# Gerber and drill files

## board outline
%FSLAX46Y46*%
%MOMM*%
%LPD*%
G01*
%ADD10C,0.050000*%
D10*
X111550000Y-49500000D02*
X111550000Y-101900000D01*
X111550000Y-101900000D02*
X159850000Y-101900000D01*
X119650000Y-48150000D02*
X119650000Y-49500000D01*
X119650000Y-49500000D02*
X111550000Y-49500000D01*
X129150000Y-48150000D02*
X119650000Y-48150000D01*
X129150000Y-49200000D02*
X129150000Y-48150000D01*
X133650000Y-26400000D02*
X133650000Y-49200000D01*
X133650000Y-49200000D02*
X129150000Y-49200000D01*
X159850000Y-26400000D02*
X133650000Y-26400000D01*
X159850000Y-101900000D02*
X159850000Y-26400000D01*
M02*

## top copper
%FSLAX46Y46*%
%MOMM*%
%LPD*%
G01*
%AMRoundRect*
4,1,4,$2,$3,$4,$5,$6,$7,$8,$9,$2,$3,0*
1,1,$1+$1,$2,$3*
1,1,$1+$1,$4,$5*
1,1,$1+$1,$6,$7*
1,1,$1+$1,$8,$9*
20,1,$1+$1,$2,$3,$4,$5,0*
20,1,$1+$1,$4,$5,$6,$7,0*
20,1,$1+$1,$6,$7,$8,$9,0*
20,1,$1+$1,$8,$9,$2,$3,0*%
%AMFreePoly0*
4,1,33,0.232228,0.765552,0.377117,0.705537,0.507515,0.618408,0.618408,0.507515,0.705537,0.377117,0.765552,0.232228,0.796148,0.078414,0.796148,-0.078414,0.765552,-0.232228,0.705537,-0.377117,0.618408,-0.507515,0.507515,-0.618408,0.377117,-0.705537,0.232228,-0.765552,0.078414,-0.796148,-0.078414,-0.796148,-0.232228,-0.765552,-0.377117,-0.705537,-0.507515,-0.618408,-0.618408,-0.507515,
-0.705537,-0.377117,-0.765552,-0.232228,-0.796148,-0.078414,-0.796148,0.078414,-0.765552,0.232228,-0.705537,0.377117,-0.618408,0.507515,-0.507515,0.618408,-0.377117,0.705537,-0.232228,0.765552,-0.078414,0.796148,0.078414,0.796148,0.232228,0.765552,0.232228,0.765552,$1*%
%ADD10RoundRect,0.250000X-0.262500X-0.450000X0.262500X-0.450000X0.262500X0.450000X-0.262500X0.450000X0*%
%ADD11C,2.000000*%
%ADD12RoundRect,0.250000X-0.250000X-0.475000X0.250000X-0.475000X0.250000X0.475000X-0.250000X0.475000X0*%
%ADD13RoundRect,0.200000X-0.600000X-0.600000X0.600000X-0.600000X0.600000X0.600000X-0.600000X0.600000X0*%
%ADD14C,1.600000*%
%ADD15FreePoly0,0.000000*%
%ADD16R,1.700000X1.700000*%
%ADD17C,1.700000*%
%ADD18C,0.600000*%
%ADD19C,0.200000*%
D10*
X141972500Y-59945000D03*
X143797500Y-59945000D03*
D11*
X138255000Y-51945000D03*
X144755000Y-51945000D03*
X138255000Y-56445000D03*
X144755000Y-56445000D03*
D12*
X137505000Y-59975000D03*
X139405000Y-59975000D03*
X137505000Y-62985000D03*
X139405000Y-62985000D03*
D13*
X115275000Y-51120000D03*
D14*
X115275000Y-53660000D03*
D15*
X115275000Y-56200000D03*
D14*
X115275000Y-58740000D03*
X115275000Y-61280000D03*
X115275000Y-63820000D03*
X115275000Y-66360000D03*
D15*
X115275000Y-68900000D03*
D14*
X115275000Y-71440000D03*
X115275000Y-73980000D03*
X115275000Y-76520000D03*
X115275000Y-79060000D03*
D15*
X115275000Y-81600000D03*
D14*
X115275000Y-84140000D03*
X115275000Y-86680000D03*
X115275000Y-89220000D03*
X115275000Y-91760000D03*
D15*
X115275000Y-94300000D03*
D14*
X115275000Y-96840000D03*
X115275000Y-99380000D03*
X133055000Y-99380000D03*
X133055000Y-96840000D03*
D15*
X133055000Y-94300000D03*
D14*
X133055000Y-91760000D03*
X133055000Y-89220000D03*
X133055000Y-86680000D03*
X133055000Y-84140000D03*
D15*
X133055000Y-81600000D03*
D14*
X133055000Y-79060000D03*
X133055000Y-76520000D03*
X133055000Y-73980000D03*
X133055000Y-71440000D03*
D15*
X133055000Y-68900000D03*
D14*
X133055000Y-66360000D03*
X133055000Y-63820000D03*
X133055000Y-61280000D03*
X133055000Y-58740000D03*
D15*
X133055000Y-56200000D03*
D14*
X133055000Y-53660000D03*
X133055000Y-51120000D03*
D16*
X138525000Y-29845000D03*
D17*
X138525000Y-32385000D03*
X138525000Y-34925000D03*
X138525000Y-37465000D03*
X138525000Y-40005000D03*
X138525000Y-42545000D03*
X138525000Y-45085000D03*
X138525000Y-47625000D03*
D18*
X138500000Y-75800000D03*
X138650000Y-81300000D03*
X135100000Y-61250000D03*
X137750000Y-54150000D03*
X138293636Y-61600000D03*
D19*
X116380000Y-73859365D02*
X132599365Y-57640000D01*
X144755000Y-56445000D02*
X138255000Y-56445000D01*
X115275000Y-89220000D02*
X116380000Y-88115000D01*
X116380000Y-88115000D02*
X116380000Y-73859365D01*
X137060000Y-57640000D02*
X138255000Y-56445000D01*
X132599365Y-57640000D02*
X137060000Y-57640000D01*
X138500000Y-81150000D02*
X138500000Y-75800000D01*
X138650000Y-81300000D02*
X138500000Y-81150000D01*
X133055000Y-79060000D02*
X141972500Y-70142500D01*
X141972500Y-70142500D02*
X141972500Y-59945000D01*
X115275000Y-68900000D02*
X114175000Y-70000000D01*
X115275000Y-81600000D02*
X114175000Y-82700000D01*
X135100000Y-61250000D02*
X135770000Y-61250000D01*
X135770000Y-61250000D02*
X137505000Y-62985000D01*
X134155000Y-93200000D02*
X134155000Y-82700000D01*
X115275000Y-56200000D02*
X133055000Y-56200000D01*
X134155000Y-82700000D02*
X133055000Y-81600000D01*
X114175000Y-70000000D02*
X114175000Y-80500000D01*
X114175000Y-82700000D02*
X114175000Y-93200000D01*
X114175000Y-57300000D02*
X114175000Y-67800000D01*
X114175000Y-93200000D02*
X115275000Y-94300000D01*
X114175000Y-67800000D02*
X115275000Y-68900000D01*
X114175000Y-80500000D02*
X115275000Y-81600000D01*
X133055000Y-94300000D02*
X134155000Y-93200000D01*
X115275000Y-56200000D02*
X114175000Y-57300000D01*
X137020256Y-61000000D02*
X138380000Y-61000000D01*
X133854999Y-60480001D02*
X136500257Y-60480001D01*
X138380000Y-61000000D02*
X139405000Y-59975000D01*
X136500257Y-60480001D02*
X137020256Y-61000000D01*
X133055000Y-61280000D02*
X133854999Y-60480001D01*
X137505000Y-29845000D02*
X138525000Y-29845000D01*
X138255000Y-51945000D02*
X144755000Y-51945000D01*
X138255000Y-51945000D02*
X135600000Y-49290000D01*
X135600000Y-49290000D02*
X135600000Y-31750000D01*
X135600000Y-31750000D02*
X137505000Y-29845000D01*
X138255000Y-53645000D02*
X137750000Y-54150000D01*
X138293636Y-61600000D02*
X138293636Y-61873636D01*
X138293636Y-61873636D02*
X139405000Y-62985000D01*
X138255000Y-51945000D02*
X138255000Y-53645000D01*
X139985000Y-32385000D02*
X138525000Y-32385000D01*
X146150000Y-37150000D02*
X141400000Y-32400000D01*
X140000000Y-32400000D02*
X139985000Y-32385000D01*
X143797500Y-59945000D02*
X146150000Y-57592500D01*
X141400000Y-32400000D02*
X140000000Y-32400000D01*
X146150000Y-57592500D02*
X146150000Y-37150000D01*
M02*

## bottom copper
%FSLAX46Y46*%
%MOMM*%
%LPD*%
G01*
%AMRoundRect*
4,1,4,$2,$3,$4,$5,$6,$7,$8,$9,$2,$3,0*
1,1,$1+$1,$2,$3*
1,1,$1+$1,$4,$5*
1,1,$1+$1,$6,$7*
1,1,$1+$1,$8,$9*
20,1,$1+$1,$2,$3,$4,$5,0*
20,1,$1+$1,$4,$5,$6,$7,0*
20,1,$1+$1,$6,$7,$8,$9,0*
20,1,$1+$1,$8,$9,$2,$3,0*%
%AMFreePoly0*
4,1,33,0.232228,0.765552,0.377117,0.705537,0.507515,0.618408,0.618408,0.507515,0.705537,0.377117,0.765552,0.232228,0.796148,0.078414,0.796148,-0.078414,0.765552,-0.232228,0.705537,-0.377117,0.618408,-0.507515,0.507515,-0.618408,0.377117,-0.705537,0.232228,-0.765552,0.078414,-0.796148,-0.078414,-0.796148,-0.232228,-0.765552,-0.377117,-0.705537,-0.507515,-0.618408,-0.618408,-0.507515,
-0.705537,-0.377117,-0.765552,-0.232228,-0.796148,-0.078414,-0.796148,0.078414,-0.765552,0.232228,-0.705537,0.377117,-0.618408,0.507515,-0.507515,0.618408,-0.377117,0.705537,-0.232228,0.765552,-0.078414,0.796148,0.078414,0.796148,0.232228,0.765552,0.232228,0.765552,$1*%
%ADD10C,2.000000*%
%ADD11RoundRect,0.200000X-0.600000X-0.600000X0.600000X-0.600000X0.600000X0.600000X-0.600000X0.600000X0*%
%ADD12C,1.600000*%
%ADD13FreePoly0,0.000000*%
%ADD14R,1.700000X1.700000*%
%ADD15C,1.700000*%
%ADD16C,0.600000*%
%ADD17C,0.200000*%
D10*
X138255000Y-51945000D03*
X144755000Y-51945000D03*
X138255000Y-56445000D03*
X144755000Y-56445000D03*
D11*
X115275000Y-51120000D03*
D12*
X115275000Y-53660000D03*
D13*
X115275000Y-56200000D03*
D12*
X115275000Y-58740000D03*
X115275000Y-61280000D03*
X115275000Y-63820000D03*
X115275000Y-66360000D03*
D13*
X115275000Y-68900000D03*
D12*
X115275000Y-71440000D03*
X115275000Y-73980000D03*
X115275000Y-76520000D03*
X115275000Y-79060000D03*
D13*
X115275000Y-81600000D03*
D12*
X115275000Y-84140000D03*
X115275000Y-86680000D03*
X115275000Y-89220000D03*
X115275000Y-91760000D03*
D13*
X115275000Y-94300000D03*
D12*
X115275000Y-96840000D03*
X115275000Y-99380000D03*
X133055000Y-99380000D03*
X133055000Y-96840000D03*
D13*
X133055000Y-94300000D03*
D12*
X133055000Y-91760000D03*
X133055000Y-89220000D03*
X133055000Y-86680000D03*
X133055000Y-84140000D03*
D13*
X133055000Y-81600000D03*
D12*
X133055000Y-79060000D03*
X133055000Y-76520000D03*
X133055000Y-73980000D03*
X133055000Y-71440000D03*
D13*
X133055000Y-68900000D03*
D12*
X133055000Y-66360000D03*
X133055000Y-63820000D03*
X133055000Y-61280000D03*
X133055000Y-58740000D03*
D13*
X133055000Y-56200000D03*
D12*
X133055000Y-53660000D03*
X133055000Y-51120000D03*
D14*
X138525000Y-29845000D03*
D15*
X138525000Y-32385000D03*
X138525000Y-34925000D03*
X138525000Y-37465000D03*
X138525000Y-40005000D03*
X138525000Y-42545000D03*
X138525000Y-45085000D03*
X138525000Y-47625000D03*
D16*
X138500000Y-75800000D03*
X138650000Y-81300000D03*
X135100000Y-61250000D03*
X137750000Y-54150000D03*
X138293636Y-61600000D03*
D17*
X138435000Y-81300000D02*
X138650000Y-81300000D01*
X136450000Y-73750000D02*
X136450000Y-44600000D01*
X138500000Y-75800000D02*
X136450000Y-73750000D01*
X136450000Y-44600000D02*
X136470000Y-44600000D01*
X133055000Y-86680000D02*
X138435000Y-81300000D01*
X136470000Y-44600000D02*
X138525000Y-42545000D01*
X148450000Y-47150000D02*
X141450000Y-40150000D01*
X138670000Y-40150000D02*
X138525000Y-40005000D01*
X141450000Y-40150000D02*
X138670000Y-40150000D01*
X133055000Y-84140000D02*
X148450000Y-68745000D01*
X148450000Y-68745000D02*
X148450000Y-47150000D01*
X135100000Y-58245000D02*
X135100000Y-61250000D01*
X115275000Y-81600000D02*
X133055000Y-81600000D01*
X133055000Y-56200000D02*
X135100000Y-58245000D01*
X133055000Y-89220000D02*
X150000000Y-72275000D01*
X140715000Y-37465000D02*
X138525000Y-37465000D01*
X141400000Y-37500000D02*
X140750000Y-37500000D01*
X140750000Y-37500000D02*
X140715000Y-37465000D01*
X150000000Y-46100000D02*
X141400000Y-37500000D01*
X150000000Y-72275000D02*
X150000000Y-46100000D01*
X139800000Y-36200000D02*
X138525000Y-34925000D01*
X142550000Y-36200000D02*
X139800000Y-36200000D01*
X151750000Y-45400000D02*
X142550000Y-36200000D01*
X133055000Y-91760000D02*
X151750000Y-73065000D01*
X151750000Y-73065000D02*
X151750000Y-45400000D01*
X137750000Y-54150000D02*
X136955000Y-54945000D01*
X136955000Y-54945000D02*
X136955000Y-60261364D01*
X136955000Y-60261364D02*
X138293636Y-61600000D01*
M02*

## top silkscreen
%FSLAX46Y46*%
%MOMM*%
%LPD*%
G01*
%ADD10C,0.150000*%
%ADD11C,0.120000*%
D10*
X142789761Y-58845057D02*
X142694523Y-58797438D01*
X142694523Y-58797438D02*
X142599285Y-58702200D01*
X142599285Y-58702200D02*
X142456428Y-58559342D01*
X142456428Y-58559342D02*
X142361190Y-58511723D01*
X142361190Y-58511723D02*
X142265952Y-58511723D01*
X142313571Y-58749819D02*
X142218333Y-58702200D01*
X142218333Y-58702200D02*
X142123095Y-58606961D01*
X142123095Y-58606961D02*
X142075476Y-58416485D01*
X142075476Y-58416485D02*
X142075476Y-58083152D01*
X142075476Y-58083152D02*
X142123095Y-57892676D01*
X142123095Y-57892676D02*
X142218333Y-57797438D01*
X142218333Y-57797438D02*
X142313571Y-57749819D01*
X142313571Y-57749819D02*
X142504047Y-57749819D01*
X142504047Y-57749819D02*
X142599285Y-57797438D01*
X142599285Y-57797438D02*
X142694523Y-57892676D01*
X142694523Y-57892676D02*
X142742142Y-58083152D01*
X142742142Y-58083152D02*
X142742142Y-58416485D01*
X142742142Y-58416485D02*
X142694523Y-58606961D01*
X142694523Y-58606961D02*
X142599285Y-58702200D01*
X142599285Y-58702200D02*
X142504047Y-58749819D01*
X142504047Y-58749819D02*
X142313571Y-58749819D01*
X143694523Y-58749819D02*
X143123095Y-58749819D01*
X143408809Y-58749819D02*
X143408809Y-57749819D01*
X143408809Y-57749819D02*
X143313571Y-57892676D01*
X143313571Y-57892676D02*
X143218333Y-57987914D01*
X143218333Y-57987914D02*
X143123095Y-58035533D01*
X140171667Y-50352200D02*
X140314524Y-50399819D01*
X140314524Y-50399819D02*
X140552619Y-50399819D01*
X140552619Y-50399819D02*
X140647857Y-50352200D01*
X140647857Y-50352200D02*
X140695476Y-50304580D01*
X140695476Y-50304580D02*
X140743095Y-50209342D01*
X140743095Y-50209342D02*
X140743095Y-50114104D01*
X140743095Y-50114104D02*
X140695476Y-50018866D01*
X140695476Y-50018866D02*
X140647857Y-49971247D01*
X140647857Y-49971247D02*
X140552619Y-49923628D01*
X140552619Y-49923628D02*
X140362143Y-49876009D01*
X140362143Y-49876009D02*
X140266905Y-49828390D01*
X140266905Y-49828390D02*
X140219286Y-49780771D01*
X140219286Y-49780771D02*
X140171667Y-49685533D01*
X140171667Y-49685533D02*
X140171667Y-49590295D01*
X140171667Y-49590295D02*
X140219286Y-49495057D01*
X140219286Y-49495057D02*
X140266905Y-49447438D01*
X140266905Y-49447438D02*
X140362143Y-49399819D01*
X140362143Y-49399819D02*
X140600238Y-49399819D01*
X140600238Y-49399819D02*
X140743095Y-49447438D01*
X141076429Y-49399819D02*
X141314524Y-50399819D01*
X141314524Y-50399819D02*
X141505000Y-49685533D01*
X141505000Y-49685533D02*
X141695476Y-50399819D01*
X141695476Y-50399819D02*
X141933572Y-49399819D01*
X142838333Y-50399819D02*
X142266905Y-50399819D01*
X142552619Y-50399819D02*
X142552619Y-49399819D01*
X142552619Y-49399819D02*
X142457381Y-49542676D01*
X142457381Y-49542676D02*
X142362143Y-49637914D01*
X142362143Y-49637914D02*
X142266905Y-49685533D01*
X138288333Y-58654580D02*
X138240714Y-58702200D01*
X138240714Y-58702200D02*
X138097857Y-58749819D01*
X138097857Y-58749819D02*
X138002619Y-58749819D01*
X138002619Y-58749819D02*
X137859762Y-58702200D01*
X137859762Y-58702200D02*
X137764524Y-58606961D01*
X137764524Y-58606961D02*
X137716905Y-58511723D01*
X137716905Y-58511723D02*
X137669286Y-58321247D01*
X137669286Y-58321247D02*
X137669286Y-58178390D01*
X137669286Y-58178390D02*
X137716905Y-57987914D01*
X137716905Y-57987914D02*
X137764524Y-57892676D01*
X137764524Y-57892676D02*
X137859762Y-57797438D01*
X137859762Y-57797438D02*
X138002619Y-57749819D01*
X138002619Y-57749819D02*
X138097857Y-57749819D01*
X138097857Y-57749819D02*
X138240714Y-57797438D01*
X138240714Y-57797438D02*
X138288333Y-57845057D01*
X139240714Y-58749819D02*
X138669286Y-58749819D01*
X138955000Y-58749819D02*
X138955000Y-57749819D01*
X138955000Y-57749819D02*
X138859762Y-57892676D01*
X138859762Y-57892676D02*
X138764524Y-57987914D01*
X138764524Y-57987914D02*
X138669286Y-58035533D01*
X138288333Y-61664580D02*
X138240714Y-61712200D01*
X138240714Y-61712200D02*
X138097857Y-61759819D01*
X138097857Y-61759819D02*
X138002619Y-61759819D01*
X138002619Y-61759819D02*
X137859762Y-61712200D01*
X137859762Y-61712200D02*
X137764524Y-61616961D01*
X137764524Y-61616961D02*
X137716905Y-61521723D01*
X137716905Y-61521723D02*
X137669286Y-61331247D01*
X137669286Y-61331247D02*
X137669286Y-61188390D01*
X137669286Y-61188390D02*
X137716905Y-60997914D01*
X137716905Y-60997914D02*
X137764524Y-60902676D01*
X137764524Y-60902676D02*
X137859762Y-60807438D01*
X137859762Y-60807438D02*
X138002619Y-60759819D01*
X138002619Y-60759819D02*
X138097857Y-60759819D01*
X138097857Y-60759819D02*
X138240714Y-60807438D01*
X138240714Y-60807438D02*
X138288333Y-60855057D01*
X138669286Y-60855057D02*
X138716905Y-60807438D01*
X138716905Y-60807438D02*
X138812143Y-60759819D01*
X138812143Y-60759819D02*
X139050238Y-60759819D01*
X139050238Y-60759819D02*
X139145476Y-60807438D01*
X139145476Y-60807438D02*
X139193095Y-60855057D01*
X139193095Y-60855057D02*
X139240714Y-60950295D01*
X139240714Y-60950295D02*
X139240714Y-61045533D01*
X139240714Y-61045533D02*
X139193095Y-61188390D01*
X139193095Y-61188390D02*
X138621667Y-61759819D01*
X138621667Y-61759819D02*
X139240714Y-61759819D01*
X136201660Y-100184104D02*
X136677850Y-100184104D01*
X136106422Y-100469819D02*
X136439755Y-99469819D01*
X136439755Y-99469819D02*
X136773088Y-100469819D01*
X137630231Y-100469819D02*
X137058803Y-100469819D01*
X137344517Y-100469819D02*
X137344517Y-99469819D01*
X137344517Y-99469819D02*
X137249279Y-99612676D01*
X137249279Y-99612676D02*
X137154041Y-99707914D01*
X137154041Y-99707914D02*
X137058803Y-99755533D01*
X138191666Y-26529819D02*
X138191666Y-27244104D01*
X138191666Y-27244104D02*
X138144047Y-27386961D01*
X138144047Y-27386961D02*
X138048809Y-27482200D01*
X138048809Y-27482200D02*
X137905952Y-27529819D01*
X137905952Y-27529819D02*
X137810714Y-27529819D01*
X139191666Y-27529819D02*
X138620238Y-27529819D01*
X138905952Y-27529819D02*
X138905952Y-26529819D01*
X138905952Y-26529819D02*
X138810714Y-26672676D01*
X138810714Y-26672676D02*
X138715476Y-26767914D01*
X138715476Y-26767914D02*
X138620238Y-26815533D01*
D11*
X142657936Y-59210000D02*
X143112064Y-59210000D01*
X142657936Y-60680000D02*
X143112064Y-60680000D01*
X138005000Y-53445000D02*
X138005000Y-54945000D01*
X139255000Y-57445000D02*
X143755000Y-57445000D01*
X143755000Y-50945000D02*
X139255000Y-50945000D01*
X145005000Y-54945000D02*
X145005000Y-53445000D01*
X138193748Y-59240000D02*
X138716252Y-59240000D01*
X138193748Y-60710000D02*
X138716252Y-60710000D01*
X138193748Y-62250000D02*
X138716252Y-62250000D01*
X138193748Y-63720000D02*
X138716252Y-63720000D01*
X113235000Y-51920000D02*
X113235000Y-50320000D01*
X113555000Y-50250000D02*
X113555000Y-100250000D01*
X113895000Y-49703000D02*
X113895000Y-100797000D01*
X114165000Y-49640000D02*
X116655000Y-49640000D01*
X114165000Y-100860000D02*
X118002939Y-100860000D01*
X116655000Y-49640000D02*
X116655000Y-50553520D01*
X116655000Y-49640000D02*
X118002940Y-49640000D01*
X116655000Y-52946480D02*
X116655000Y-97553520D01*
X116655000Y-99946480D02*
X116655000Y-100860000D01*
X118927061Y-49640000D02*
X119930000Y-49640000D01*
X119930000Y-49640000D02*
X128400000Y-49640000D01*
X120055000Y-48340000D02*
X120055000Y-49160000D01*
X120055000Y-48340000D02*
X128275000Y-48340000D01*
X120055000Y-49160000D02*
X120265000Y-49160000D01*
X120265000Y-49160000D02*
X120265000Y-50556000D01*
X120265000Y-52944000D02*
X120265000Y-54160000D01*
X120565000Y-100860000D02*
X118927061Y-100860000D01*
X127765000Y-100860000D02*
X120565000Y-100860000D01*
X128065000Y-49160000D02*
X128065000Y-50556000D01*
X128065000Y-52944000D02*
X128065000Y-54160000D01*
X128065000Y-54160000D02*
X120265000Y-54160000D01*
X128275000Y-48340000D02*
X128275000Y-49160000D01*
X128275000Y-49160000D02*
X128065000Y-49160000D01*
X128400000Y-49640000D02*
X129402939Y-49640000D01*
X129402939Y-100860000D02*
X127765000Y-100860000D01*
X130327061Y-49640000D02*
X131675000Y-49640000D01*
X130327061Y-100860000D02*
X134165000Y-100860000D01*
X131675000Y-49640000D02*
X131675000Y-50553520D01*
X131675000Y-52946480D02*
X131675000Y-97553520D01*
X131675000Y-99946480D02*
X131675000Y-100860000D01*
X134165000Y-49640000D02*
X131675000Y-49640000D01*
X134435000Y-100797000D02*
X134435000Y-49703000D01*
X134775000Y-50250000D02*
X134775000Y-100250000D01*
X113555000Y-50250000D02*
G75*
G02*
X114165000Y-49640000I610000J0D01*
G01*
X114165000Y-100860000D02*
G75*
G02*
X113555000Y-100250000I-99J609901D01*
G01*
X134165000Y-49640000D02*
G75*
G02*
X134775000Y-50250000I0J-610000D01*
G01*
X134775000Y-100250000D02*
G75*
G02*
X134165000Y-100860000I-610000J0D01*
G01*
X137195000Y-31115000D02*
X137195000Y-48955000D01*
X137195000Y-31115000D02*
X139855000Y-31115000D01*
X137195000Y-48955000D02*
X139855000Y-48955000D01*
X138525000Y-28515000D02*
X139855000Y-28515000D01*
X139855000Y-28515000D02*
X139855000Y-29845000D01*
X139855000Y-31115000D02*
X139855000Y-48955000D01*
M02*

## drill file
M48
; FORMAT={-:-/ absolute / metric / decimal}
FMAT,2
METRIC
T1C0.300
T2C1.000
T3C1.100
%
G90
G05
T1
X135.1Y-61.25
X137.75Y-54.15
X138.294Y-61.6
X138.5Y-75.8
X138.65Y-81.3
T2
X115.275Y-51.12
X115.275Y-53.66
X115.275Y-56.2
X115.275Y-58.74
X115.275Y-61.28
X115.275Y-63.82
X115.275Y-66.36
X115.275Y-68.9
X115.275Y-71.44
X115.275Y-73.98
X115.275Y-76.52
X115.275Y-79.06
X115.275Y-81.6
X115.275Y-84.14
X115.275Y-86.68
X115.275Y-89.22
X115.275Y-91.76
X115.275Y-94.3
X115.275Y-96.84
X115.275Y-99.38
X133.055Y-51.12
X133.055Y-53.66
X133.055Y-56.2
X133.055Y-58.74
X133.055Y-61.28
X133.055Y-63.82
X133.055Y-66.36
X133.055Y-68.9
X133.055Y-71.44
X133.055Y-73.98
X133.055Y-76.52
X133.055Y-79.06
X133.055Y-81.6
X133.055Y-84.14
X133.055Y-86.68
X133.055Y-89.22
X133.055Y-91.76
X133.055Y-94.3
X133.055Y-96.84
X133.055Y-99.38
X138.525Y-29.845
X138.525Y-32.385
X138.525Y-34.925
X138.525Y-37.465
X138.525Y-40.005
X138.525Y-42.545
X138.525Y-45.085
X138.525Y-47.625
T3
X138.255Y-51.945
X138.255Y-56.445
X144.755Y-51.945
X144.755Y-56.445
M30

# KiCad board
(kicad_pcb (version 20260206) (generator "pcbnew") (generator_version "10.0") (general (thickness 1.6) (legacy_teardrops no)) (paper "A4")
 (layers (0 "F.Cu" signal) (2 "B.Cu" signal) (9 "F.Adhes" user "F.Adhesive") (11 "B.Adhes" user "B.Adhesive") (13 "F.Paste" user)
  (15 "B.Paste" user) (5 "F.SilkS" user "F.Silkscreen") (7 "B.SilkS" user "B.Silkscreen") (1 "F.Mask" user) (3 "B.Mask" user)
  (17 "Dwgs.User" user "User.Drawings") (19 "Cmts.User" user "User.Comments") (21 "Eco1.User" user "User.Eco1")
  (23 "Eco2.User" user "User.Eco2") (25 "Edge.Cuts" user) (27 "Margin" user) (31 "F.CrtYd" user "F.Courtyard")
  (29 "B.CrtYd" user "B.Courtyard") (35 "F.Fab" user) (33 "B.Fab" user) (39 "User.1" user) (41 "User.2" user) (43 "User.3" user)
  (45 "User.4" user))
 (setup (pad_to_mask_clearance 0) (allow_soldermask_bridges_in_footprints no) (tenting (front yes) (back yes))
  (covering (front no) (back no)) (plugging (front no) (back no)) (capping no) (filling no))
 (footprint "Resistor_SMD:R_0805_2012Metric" (layer "F.Cu") (at 142.885 59.945)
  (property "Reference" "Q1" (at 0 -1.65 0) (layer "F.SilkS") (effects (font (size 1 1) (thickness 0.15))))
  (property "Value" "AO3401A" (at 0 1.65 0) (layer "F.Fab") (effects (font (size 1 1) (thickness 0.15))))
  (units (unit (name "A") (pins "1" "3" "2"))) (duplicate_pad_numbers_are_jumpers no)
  (fp_line (start -0.227064 -0.735) (end 0.227064 -0.735) (stroke (width 0.12) (type solid)) (layer "F.SilkS"))
  (fp_line (start -0.227064 0.735) (end 0.227064 0.735) (stroke (width 0.12) (type solid)) (layer "F.SilkS"))
  (pad "1" smd roundrect (at -0.9125 0) (size 1.025 1.4) (layers "F.Cu" "F.Mask" "F.Paste") (roundrect_rratio 0.243902) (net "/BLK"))
  (pad "2" smd roundrect (at 0.9125 0) (size 1.025 1.4) (layers "F.Cu" "F.Mask" "F.Paste") (roundrect_rratio 0.243902) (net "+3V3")))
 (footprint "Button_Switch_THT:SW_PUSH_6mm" (layer "F.Cu") (at 138.255 51.945)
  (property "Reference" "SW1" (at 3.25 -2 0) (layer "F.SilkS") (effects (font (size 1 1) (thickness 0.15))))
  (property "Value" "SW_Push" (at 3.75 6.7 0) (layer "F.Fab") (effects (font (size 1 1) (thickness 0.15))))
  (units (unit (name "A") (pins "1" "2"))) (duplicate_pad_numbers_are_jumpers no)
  (fp_line (start -0.25 1.5) (end -0.25 3) (stroke (width 0.12) (type solid)) (layer "F.SilkS"))
  (fp_line (start 1 5.5) (end 5.5 5.5) (stroke (width 0.12) (type solid)) (layer "F.SilkS"))
  (fp_line (start 5.5 -1) (end 1 -1) (stroke (width 0.12) (type solid)) (layer "F.SilkS"))
  (fp_line (start 6.75 3) (end 6.75 1.5) (stroke (width 0.12) (type solid)) (layer "F.SilkS"))
  (pad "1" thru_hole circle (at 0 0 90) (size 2 2) (drill 1.1) (layers "*.Cu" "*.Mask") (remove_unused_layers no) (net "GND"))
  (pad "1" thru_hole circle (at 6.5 0 90) (size 2 2) (drill 1.1) (layers "*.Cu" "*.Mask") (remove_unused_layers no) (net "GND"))
  (pad "2" thru_hole circle (at 0 4.5 90) (size 2 2) (drill 1.1) (layers "*.Cu" "*.Mask") (remove_unused_layers no) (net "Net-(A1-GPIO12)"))
  (pad "2" thru_hole circle (at 6.5 4.5 90) (size 2 2) (drill 1.1) (layers "*.Cu" "*.Mask") (remove_unused_layers no)
   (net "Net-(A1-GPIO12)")))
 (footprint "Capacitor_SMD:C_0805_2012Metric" (layer "F.Cu") (at 138.455 59.975)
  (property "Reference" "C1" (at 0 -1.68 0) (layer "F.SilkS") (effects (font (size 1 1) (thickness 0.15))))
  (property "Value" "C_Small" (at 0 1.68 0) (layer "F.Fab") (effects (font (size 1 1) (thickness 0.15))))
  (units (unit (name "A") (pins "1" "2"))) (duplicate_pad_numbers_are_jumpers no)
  (fp_line (start -0.261252 -0.735) (end 0.261252 -0.735) (stroke (width 0.12) (type solid)) (layer "F.SilkS"))
  (fp_line (start -0.261252 0.735) (end 0.261252 0.735) (stroke (width 0.12) (type solid)) (layer "F.SilkS"))
  (pad "1" smd roundrect (at -0.95 0) (size 1 1.45) (layers "F.Cu" "F.Mask" "F.Paste") (roundrect_rratio 0.25) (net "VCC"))
  (pad "2" smd roundrect (at 0.95 0) (size 1 1.45) (layers "F.Cu" "F.Mask" "F.Paste") (roundrect_rratio 0.25) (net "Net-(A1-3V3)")))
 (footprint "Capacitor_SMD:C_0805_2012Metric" (layer "F.Cu") (at 138.455 62.985)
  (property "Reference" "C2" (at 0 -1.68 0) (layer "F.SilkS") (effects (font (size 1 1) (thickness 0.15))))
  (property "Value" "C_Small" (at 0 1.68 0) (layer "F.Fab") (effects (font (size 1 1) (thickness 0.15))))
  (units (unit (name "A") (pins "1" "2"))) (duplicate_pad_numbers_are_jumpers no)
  (fp_line (start -0.261252 -0.735) (end 0.261252 -0.735) (stroke (width 0.12) (type solid)) (layer "F.SilkS"))
  (fp_line (start -0.261252 0.735) (end 0.261252 0.735) (stroke (width 0.12) (type solid)) (layer "F.SilkS"))
  (pad "1" smd roundrect (at -0.95 0) (size 1 1.45) (layers "F.Cu" "F.Mask" "F.Paste") (roundrect_rratio 0.25) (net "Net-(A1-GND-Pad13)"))
  (pad "2" smd roundrect (at 0.95 0) (size 1 1.45) (layers "F.Cu" "F.Mask" "F.Paste") (roundrect_rratio 0.25) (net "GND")))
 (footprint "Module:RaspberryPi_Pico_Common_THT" (layer "F.Cu") (at 115.275 51.12)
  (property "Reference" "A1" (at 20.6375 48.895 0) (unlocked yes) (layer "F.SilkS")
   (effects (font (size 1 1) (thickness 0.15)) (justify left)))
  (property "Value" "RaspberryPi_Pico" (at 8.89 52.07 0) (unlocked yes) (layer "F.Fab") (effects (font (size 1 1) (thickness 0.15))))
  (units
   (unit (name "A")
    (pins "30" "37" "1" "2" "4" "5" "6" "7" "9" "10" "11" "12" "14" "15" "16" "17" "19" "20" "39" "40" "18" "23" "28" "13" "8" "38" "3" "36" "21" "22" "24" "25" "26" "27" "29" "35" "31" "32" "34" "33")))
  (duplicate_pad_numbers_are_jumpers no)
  (fp_line (start -2.04 0.8) (end -2.04 -0.8) (stroke (width 0.12) (type solid)) (layer "F.SilkS"))
  (fp_line (start -1.72 -0.87) (end -1.72 49.13) (stroke (width 0.12) (type solid)) (layer "F.SilkS"))
  (fp_line (start -1.38 -1.417) (end -1.38 49.677) (stroke (width 0.12) (type solid)) (layer "F.SilkS"))
  (fp_line (start -1.11 -1.48) (end 1.38 -1.48) (stroke (width 0.12) (type solid)) (layer "F.SilkS"))
  (fp_line (start -1.11 49.74) (end 2.727939 49.74) (stroke (width 0.12) (type solid)) (layer "F.SilkS"))
  (fp_line (start 1.38 -1.48) (end 1.38 -0.56648) (stroke (width 0.12) (type solid)) (layer "F.SilkS"))
  (fp_line (start 1.38 -1.48) (end 2.72794 -1.48) (stroke (width 0.12) (type solid)) (layer "F.SilkS"))
  (fp_line (start 1.38 1.82648) (end 1.38 46.43352) (stroke (width 0.12) (type solid)) (layer "F.SilkS"))
  (fp_line (start 1.38 48.82648) (end 1.38 49.74) (stroke (width 0.12) (type solid)) (layer "F.SilkS"))
  (fp_line (start 3.652061 -1.48) (end 4.655 -1.48) (stroke (width 0.12) (type solid)) (layer "F.SilkS"))
  (fp_line (start 4.655 -1.48) (end 13.125 -1.48) (stroke (width 0.12) (type solid)) (layer "F.SilkS"))
  (fp_line (start 4.78 -2.78) (end 4.78 -1.96) (stroke (width 0.12) (type solid)) (layer "F.SilkS"))
  (fp_line (start 4.78 -2.78) (end 13 -2.78) (stroke (width 0.12) (type solid)) (layer "F.SilkS"))
  (fp_line (start 4.78 -1.96) (end 4.99 -1.96) (stroke (width 0.12) (type solid)) (layer "F.SilkS"))
  (fp_line (start 4.99 -1.96) (end 4.99 -0.564) (stroke (width 0.12) (type solid)) (layer "F.SilkS"))
  (fp_line (start 4.99 1.824) (end 4.99 3.04) (stroke (width 0.12) (type solid)) (layer "F.SilkS"))
  (fp_line (start 5.29 49.74) (end 3.652061 49.74) (stroke (width 0.12) (type solid)) (layer "F.SilkS"))
  (fp_line (start 12.49 49.74) (end 5.29 49.74) (stroke (width 0.12) (type solid)) (layer "F.SilkS"))
  (fp_line (start 12.79 -1.96) (end 12.79 -0.564) (stroke (width 0.12) (type solid)) (layer "F.SilkS"))
  (fp_line (start 12.79 1.824) (end 12.79 3.04) (stroke (width 0.12) (type solid)) (layer "F.SilkS"))
  (fp_line (start 12.79 3.04) (end 4.99 3.04) (stroke (width 0.12) (type solid)) (layer "F.SilkS"))
  (fp_line (start 13 -2.78) (end 13 -1.96) (stroke (width 0.12) (type solid)) (layer "F.SilkS"))
  (fp_line (start 13 -1.96) (end 12.79 -1.96) (stroke (width 0.12) (type solid)) (layer "F.SilkS"))
  (fp_line (start 13.125 -1.48) (end 14.127939 -1.48) (stroke (width 0.12) (type solid)) (layer "F.SilkS"))
  (fp_line (start 14.127939 49.74) (end 12.49 49.74) (stroke (width 0.12) (type solid)) (layer "F.SilkS"))
  (fp_line (start 15.052061 -1.48) (end 16.4 -1.48) (stroke (width 0.12) (type solid)) (layer "F.SilkS"))
  (fp_line (start 15.052061 49.74) (end 18.89 49.74) (stroke (width 0.12) (type solid)) (layer "F.SilkS"))
  (fp_line (start 16.4 -1.48) (end 16.4 -0.56648) (stroke (width 0.12) (type solid)) (layer "F.SilkS"))
  (fp_line (start 16.4 1.82648) (end 16.4 46.43352) (stroke (width 0.12) (type solid)) (layer "F.SilkS"))
  (fp_line (start 16.4 48.82648) (end 16.4 49.74) (stroke (width 0.12) (type solid)) (layer "F.SilkS"))
  (fp_line (start 18.89 -1.48) (end 16.4 -1.48) (stroke (width 0.12) (type solid)) (layer "F.SilkS"))
  (fp_line (start 19.16 49.677) (end 19.16 -1.417) (stroke (width 0.12) (type solid)) (layer "F.SilkS"))
  (fp_line (start 19.5 -0.87) (end 19.5 49.13) (stroke (width 0.12) (type solid)) (layer "F.SilkS"))
  (fp_arc (start -1.72 -0.87) (mid -1.541335 -1.301335) (end -1.11 -1.48) (stroke (width 0.12) (type solid)) (layer "F.SilkS"))
  (fp_arc (start -1.11 49.74) (mid -1.541364 49.561364) (end -1.72 49.13) (stroke (width 0.12) (type solid)) (layer "F.SilkS"))
  (fp_arc (start 18.89 -1.48) (mid 19.321335 -1.301335) (end 19.5 -0.87) (stroke (width 0.12) (type solid)) (layer "F.SilkS"))
  (fp_arc (start 19.5 49.13) (mid 19.321335 49.561335) (end 18.89 49.74) (stroke (width 0.12) (type solid)) (layer "F.SilkS"))
  (pad "1" thru_hole roundrect (at 0 0) (size 1.6 1.6) (drill 1) (layers "*.Cu" "*.Mask") (remove_unused_layers no) (roundrect_rratio 0.125)
   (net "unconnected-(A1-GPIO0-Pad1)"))
  (pad "2" thru_hole circle (at 0 2.54) (size 1.6 1.6) (drill 1) (layers "*.Cu" "*.Mask") (remove_unused_layers no)
   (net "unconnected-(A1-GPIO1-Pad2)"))
  (pad "3" thru_hole custom (at 0 5.08) (size 1.6 1.6) (drill 1) (layers "*.Cu" "*.Mask") (remove_unused_layers no)
   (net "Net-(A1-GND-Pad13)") (options (clearance outline) (anchor circle)) (primitives))
  (pad "4" thru_hole circle (at 0 7.62) (size 1.6 1.6) (drill 1) (layers "*.Cu" "*.Mask") (remove_unused_layers no)
   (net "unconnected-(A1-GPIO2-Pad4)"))
  (pad "5" thru_hole circle (at 0 10.16) (size 1.6 1.6) (drill 1) (layers "*.Cu" "*.Mask") (remove_unused_layers no)
   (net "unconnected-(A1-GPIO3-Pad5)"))
  (pad "6" thru_hole circle (at 0 12.7) (size 1.6 1.6) (drill 1) (layers "*.Cu" "*.Mask") (remove_unused_layers no)
   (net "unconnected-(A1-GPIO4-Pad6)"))
  (pad "7" thru_hole circle (at 0 15.24) (size 1.6 1.6) (drill 1) (layers "*.Cu" "*.Mask") (remove_unused_layers no)
   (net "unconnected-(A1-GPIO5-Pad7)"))
  (pad "8" thru_hole custom (at 0 17.78) (size 1.6 1.6) (drill 1) (layers "*.Cu" "*.Mask") (remove_unused_layers no)
   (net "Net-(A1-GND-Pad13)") (options (clearance outline) (anchor circle)) (primitives))
  (pad "9" thru_hole circle (at 0 20.32) (size 1.6 1.6) (drill 1) (layers "*.Cu" "*.Mask") (remove_unused_layers no)
   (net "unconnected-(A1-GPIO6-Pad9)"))
  (pad "10" thru_hole circle (at 0 22.86) (size 1.6 1.6) (drill 1) (layers "*.Cu" "*.Mask") (remove_unused_layers no)
   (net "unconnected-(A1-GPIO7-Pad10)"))
  (pad "11" thru_hole circle (at 0 25.4) (size 1.6 1.6) (drill 1) (layers "*.Cu" "*.Mask") (remove_unused_layers no)
   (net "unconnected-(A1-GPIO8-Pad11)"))
  (pad "12" thru_hole circle (at 0 27.94) (size 1.6 1.6) (drill 1) (layers "*.Cu" "*.Mask") (remove_unused_layers no)
   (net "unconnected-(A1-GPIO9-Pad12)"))
  (pad "13" thru_hole custom (at 0 30.48) (size 1.6 1.6) (drill 1) (layers "*.Cu" "*.Mask") (remove_unused_layers no)
   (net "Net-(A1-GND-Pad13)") (options (clearance outline) (anchor circle)) (primitives))
  (pad "14" thru_hole circle (at 0 33.02) (size 1.6 1.6) (drill 1) (layers "*.Cu" "*.Mask") (remove_unused_layers no)
   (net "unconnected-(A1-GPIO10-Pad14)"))
  (pad "15" thru_hole circle (at 0 35.56) (size 1.6 1.6) (drill 1) (layers "*.Cu" "*.Mask") (remove_unused_layers no)
   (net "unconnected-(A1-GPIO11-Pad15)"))
  (pad "16" thru_hole circle (at 0 38.1) (size 1.6 1.6) (drill 1) (layers "*.Cu" "*.Mask") (remove_unused_layers no) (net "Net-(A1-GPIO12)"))
  (pad "17" thru_hole circle (at 0 40.64) (size 1.6 1.6) (drill 1) (layers "*.Cu" "*.Mask") (remove_unused_layers no)
   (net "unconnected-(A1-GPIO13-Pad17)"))
  (pad "18" thru_hole custom (at 0 43.18) (size 1.6 1.6) (drill 1) (layers "*.Cu" "*.Mask") (remove_unused_layers no)
   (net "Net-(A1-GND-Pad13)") (options (clearance outline) (anchor circle)) (primitives))
  (pad "19" thru_hole circle (at 0 45.72) (size 1.6 1.6) (drill 1) (layers "*.Cu" "*.Mask") (remove_unused_layers no)
   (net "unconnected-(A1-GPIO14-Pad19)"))
  (pad "20" thru_hole circle (at 0 48.26) (size 1.6 1.6) (drill 1) (layers "*.Cu" "*.Mask") (remove_unused_layers no)
   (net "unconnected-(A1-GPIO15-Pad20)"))
  (pad "21" thru_hole circle (at 17.78 48.26) (size 1.6 1.6) (drill 1) (layers "*.Cu" "*.Mask") (remove_unused_layers no)
   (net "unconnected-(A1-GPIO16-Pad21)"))
  (pad "22" thru_hole circle (at 17.78 45.72) (size 1.6 1.6) (drill 1) (layers "*.Cu" "*.Mask") (remove_unused_layers no)
   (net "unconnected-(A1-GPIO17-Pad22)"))
  (pad "23" thru_hole custom (at 17.78 43.18) (size 1.6 1.6) (drill 1) (layers "*.Cu" "*.Mask") (remove_unused_layers no)
   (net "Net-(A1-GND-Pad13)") (options (clearance outline) (anchor circle)) (primitives))
  (pad "24" thru_hole circle (at 17.78 40.64) (size 1.6 1.6) (drill 1) (layers "*.Cu" "*.Mask") (remove_unused_layers no) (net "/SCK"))
  (pad "25" thru_hole circle (at 17.78 38.1) (size 1.6 1.6) (drill 1) (layers "*.Cu" "*.Mask") (remove_unused_layers no) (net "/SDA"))
  (pad "26" thru_hole circle (at 17.78 35.56) (size 1.6 1.6) (drill 1) (layers "*.Cu" "*.Mask") (remove_unused_layers no) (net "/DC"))
  (pad "27" thru_hole circle (at 17.78 33.02) (size 1.6 1.6) (drill 1) (layers "*.Cu" "*.Mask") (remove_unused_layers no) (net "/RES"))
  (pad "28" thru_hole custom (at 17.78 30.48) (size 1.6 1.6) (drill 1) (layers "*.Cu" "*.Mask") (remove_unused_layers no)
   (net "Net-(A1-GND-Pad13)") (options (clearance outline) (anchor circle)) (primitives))
  (pad "29" thru_hole circle (at 17.78 27.94) (size 1.6 1.6) (drill 1) (layers "*.Cu" "*.Mask") (remove_unused_layers no) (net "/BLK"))
  (pad "30" thru_hole circle (at 17.78 25.4) (size 1.6 1.6) (drill 1) (layers "*.Cu" "*.Mask") (remove_unused_layers no)
   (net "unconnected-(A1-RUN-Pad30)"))
  (pad "31" thru_hole circle (at 17.78 22.86) (size 1.6 1.6) (drill 1) (layers "*.Cu" "*.Mask") (remove_unused_layers no)
   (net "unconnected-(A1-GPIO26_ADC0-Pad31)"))
  (pad "32" thru_hole circle (at 17.78 20.32) (size 1.6 1.6) (drill 1) (layers "*.Cu" "*.Mask") (remove_unused_layers no)
   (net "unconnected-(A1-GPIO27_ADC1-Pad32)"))
  (pad "33" thru_hole custom (at 17.78 17.78) (size 1.6 1.6) (drill 1) (layers "*.Cu" "*.Mask") (remove_unused_layers no)
   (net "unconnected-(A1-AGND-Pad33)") (options (clearance outline) (anchor circle)) (primitives))
  (pad "34" thru_hole circle (at 17.78 15.24) (size 1.6 1.6) (drill 1) (layers "*.Cu" "*.Mask") (remove_unused_layers no)
   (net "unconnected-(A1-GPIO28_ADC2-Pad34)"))
  (pad "35" thru_hole circle (at 17.78 12.7) (size 1.6 1.6) (drill 1) (layers "*.Cu" "*.Mask") (remove_unused_layers no)
   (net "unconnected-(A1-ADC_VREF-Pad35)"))
  (pad "36" thru_hole circle (at 17.78 10.16) (size 1.6 1.6) (drill 1) (layers "*.Cu" "*.Mask") (remove_unused_layers no)
   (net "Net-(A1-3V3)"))
  (pad "37" thru_hole circle (at 17.78 7.62) (size 1.6 1.6) (drill 1) (layers "*.Cu" "*.Mask") (remove_unused_layers no)
   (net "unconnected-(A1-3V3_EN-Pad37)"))
  (pad "38" thru_hole custom (at 17.78 5.08) (size 1.6 1.6) (drill 1) (layers "*.Cu" "*.Mask") (remove_unused_layers no)
   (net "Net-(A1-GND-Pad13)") (options (clearance outline) (anchor circle)) (primitives))
  (pad "39" thru_hole circle (at 17.78 2.54) (size 1.6 1.6) (drill 1) (layers "*.Cu" "*.Mask") (remove_unused_layers no)
   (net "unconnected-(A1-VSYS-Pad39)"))
  (pad "40" thru_hole circle (at 17.78 0) (size 1.6 1.6) (drill 1) (layers "*.Cu" "*.Mask") (remove_unused_layers no)
   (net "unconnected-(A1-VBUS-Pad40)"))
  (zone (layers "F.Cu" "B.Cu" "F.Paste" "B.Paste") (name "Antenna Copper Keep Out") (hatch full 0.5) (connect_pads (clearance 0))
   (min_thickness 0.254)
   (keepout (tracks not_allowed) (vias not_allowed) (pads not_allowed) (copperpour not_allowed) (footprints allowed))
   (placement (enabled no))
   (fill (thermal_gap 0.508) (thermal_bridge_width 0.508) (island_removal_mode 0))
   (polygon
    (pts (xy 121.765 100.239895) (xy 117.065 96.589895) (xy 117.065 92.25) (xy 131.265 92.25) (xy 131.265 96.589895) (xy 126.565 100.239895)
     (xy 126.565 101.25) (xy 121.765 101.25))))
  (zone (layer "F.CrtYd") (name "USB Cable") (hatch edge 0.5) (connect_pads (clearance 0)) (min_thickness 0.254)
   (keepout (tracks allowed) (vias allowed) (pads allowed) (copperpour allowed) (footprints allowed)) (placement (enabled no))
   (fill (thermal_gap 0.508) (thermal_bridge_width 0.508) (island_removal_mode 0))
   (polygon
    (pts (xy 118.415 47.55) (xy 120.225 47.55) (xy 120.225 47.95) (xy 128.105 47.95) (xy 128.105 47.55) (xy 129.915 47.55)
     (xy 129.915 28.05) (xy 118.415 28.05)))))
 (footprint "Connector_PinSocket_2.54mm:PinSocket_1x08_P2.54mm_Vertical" (layer "F.Cu") (at 138.525 29.845)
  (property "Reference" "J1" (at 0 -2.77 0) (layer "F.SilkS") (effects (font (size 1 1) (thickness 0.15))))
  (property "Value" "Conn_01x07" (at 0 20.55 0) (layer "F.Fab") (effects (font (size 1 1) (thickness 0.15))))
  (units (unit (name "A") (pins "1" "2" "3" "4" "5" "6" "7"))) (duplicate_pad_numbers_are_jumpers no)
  (fp_line (start -1.33 1.27) (end -1.33 19.11) (stroke (width 0.12) (type solid)) (layer "F.SilkS"))
  (fp_line (start -1.33 1.27) (end 1.33 1.27) (stroke (width 0.12) (type solid)) (layer "F.SilkS"))
  (fp_line (start -1.33 19.11) (end 1.33 19.11) (stroke (width 0.12) (type solid)) (layer "F.SilkS"))
  (fp_line (start 0 -1.33) (end 1.33 -1.33) (stroke (width 0.12) (type solid)) (layer "F.SilkS"))
  (fp_line (start 1.33 -1.33) (end 1.33 0) (stroke (width 0.12) (type solid)) (layer "F.SilkS"))
  (fp_line (start 1.33 1.27) (end 1.33 19.11) (stroke (width 0.12) (type solid)) (layer "F.SilkS"))
  (pad "1" thru_hole rect (at 0 0) (size 1.7 1.7) (drill 1) (layers "*.Cu" "*.Mask") (remove_unused_layers no) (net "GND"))
  (pad "2" thru_hole circle (at 0 2.54) (size 1.7 1.7) (drill 1) (layers "*.Cu" "*.Mask") (remove_unused_layers no) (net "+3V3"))
  (pad "3" thru_hole circle (at 0 5.08) (size 1.7 1.7) (drill 1) (layers "*.Cu" "*.Mask") (remove_unused_layers no) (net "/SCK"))
  (pad "4" thru_hole circle (at 0 7.62) (size 1.7 1.7) (drill 1) (layers "*.Cu" "*.Mask") (remove_unused_layers no) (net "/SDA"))
  (pad "5" thru_hole circle (at 0 10.16) (size 1.7 1.7) (drill 1) (layers "*.Cu" "*.Mask") (remove_unused_layers no) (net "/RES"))
  (pad "6" thru_hole circle (at 0 12.7) (size 1.7 1.7) (drill 1) (layers "*.Cu" "*.Mask") (remove_unused_layers no) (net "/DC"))
  (pad "7" thru_hole circle (at 0 15.24) (size 1.7 1.7) (drill 1) (layers "*.Cu" "*.Mask") (remove_unused_layers no) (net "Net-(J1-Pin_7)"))
  (pad "8" thru_hole circle (at 0 17.78) (size 1.7 1.7) (drill 1) (layers "*.Cu" "*.Mask") (remove_unused_layers no)))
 (gr_line (start 111.55 49.5) (end 111.55 101.9) (stroke (width 0.05) (type default)) (layer "Edge.Cuts"))
 (gr_line (start 111.55 101.9) (end 159.85 101.9) (stroke (width 0.05) (type default)) (layer "Edge.Cuts"))
 (gr_line (start 119.65 48.15) (end 119.65 49.5) (stroke (width 0.05) (type default)) (layer "Edge.Cuts"))
 (gr_line (start 119.65 49.5) (end 111.55 49.5) (stroke (width 0.05) (type default)) (layer "Edge.Cuts"))
 (gr_line (start 129.15 48.15) (end 119.65 48.15) (stroke (width 0.05) (type default)) (layer "Edge.Cuts"))
 (gr_line (start 129.15 49.2) (end 129.15 48.15) (stroke (width 0.05) (type default)) (layer "Edge.Cuts"))
 (gr_line (start 133.65 26.4) (end 133.65 49.2) (stroke (width 0.05) (type default)) (layer "Edge.Cuts"))
 (gr_line (start 133.65 49.2) (end 129.15 49.2) (stroke (width 0.05) (type default)) (layer "Edge.Cuts"))
 (gr_line (start 159.85 26.4) (end 133.65 26.4) (stroke (width 0.05) (type default)) (layer "Edge.Cuts"))
 (gr_line (start 159.85 101.9) (end 159.85 26.4) (stroke (width 0.05) (type default)) (layer "Edge.Cuts"))
 (segment (start 116.38 73.859365) (end 132.599365 57.64) (width 0.2) (layer "F.Cu") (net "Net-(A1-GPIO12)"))
 (segment (start 144.755 56.445) (end 138.255 56.445) (width 0.2) (layer "F.Cu") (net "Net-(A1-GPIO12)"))
 (segment (start 115.275 89.22) (end 116.38 88.115) (width 0.2) (layer "F.Cu") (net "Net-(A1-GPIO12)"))
 (segment (start 116.38 88.115) (end 116.38 73.859365) (width 0.2) (layer "F.Cu") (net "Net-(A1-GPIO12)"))
 (segment (start 137.06 57.64) (end 138.255 56.445) (width 0.2) (layer "F.Cu") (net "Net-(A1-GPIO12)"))
 (segment (start 132.599365 57.64) (end 137.06 57.64) (width 0.2) (layer "F.Cu") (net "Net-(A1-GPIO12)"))
 (segment (start 138.5 81.15) (end 138.5 75.8) (width 0.2) (layer "F.Cu") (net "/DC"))
 (segment (start 138.65 81.3) (end 138.5 81.15) (width 0.2) (layer "F.Cu") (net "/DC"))
 (via (at 138.5 75.8) (size 0.6) (drill 0.3) (layers "F.Cu" "B.Cu") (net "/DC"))
 (via (at 138.65 81.3) (size 0.6) (drill 0.3) (layers "F.Cu" "B.Cu") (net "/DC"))
 (segment (start 138.435 81.3) (end 138.65 81.3) (width 0.2) (layer "B.Cu") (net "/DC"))
 (segment (start 136.45 73.75) (end 136.45 44.6) (width 0.2) (layer "B.Cu") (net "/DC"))
 (segment (start 138.5 75.8) (end 136.45 73.75) (width 0.2) (layer "B.Cu") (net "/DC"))
 (segment (start 136.45 44.6) (end 136.47 44.6) (width 0.2) (layer "B.Cu") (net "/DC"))
 (segment (start 133.055 86.68) (end 138.435 81.3) (width 0.2) (layer "B.Cu") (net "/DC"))
 (segment (start 136.47 44.6) (end 138.525 42.545) (width 0.2) (layer "B.Cu") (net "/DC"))
 (segment (start 133.055 79.06) (end 141.9725 70.1425) (width 0.2) (layer "F.Cu") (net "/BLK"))
 (segment (start 141.9725 70.1425) (end 141.9725 59.945) (width 0.2) (layer "F.Cu") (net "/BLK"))
 (segment (start 148.45 47.15) (end 141.45 40.15) (width 0.2) (layer "B.Cu") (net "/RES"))
 (segment (start 138.67 40.15) (end 138.525 40.005) (width 0.2) (layer "B.Cu") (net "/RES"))
 (segment (start 141.45 40.15) (end 138.67 40.15) (width 0.2) (layer "B.Cu") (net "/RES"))
 (segment (start 133.055 84.14) (end 148.45 68.745) (width 0.2) (layer "B.Cu") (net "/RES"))
 (segment (start 148.45 68.745) (end 148.45 47.15) (width 0.2) (layer "B.Cu") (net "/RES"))
 (segment (start 115.275 68.9) (end 114.175 70) (width 0.2) (layer "F.Cu") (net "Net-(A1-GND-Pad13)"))
 (segment (start 115.275 81.6) (end 114.175 82.7) (width 0.2) (layer "F.Cu") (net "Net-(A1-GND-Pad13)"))
 (segment (start 135.1 61.25) (end 135.77 61.25) (width 0.2) (layer "F.Cu") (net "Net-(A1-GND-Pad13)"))
 (segment (start 135.77 61.25) (end 137.505 62.985) (width 0.2) (layer "F.Cu") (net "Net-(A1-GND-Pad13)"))
 (segment (start 134.155 93.2) (end 134.155 82.7) (width 0.2) (layer "F.Cu") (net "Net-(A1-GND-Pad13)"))
 (segment (start 115.275 56.2) (end 133.055 56.2) (width 0.2) (layer "F.Cu") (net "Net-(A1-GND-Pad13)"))
 (segment (start 134.155 82.7) (end 133.055 81.6) (width 0.2) (layer "F.Cu") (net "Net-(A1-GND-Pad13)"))
 (segment (start 114.175 70) (end 114.175 80.5) (width 0.2) (layer "F.Cu") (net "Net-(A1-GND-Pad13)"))
 (segment (start 114.175 82.7) (end 114.175 93.2) (width 0.2) (layer "F.Cu") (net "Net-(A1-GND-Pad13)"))
 (segment (start 114.175 57.3) (end 114.175 67.8) (width 0.2) (layer "F.Cu") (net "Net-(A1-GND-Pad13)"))
 (segment (start 114.175 93.2) (end 115.275 94.3) (width 0.2) (layer "F.Cu") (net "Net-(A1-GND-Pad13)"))
 (segment (start 114.175 67.8) (end 115.275 68.9) (width 0.2) (layer "F.Cu") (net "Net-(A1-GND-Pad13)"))
 (segment (start 114.175 80.5) (end 115.275 81.6) (width 0.2) (layer "F.Cu") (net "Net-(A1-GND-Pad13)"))
 (segment (start 133.055 94.3) (end 134.155 93.2) (width 0.2) (layer "F.Cu") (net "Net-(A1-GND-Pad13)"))
 (segment (start 115.275 56.2) (end 114.175 57.3) (width 0.2) (layer "F.Cu") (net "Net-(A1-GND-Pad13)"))
 (via (at 135.1 61.25) (size 0.6) (drill 0.3) (layers "F.Cu" "B.Cu") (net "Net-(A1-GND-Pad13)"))
 (segment (start 135.1 58.245) (end 135.1 61.25) (width 0.2) (layer "B.Cu") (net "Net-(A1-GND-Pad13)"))
 (segment (start 115.275 81.6) (end 133.055 81.6) (width 0.2) (layer "B.Cu") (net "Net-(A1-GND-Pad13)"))
 (segment (start 133.055 56.2) (end 135.1 58.245) (width 0.2) (layer "B.Cu") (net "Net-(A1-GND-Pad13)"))
 (segment (start 137.020256 61) (end 138.38 61) (width 0.2) (layer "F.Cu") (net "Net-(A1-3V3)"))
 (segment (start 133.854999 60.480001) (end 136.500257 60.480001) (width 0.2) (layer "F.Cu") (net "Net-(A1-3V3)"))
 (segment (start 138.38 61) (end 139.405 59.975) (width 0.2) (layer "F.Cu") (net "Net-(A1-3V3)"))
 (segment (start 136.500257 60.480001) (end 137.020256 61) (width 0.2) (layer "F.Cu") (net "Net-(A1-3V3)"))
 (segment (start 133.055 61.28) (end 133.854999 60.480001) (width 0.2) (layer "F.Cu") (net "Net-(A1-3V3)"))
 (segment (start 133.055 89.22) (end 150 72.275) (width 0.2) (layer "B.Cu") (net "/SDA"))
 (segment (start 140.715 37.465) (end 138.525 37.465) (width 0.2) (layer "B.Cu") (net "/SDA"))
 (segment (start 141.4 37.5) (end 140.75 37.5) (width 0.2) (layer "B.Cu") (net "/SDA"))
 (segment (start 140.75 37.5) (end 140.715 37.465) (width 0.2) (layer "B.Cu") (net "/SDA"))
 (segment (start 150 46.1) (end 141.4 37.5) (width 0.2) (layer "B.Cu") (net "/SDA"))
 (segment (start 150 72.275) (end 150 46.1) (width 0.2) (layer "B.Cu") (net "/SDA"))
 (segment (start 139.8 36.2) (end 138.525 34.925) (width 0.2) (layer "B.Cu") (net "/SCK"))
 (segment (start 142.55 36.2) (end 139.8 36.2) (width 0.2) (layer "B.Cu") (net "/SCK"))
 (segment (start 151.75 45.4) (end 142.55 36.2) (width 0.2) (layer "B.Cu") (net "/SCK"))
 (segment (start 133.055 91.76) (end 151.75 73.065) (width 0.2) (layer "B.Cu") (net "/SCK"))
 (segment (start 151.75 73.065) (end 151.75 45.4) (width 0.2) (layer "B.Cu") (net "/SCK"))
 (segment (start 137.505 29.845) (end 138.525 29.845) (width 0.2) (layer "F.Cu") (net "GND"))
 (segment (start 138.255 51.945) (end 144.755 51.945) (width 0.2) (layer "F.Cu") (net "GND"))
 (segment (start 138.255 51.945) (end 135.6 49.29) (width 0.2) (layer "F.Cu") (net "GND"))
 (segment (start 135.6 49.29) (end 135.6 31.75) (width 0.2) (layer "F.Cu") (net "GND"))
 (segment (start 135.6 31.75) (end 137.505 29.845) (width 0.2) (layer "F.Cu") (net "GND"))
 (segment (start 138.255 53.645) (end 137.75 54.15) (width 0.2) (layer "F.Cu") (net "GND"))
 (segment (start 138.293636 61.6) (end 138.293636 61.873636) (width 0.2) (layer "F.Cu") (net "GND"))
 (segment (start 138.293636 61.873636) (end 139.405 62.985) (width 0.2) (layer "F.Cu") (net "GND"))
 (segment (start 138.255 51.945) (end 138.255 53.645) (width 0.2) (layer "F.Cu") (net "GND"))
 (via (at 137.75 54.15) (size 0.6) (drill 0.3) (layers "F.Cu" "B.Cu") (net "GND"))
 (via (at 138.293636 61.6) (size 0.6) (drill 0.3) (layers "F.Cu" "B.Cu") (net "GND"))
 (segment (start 137.75 54.15) (end 136.955 54.945) (width 0.2) (layer "B.Cu") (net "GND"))
 (segment (start 136.955 54.945) (end 136.955 60.261364) (width 0.2) (layer "B.Cu") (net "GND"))
 (segment (start 136.955 60.261364) (end 138.293636 61.6) (width 0.2) (layer "B.Cu") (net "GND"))
 (segment (start 139.985 32.385) (end 138.525 32.385) (width 0.2) (layer "F.Cu") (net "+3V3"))
 (segment (start 146.15 37.15) (end 141.4 32.4) (width 0.2) (layer "F.Cu") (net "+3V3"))
 (segment (start 140 32.4) (end 139.985 32.385) (width 0.2) (layer "F.Cu") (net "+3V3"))
 (segment (start 143.7975 59.945) (end 146.15 57.5925) (width 0.2) (layer "F.Cu") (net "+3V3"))
 (segment (start 141.4 32.4) (end 140 32.4) (width 0.2) (layer "F.Cu") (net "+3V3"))
 (segment (start 146.15 57.5925) (end 146.15 37.15) (width 0.2) (layer "F.Cu") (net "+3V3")))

